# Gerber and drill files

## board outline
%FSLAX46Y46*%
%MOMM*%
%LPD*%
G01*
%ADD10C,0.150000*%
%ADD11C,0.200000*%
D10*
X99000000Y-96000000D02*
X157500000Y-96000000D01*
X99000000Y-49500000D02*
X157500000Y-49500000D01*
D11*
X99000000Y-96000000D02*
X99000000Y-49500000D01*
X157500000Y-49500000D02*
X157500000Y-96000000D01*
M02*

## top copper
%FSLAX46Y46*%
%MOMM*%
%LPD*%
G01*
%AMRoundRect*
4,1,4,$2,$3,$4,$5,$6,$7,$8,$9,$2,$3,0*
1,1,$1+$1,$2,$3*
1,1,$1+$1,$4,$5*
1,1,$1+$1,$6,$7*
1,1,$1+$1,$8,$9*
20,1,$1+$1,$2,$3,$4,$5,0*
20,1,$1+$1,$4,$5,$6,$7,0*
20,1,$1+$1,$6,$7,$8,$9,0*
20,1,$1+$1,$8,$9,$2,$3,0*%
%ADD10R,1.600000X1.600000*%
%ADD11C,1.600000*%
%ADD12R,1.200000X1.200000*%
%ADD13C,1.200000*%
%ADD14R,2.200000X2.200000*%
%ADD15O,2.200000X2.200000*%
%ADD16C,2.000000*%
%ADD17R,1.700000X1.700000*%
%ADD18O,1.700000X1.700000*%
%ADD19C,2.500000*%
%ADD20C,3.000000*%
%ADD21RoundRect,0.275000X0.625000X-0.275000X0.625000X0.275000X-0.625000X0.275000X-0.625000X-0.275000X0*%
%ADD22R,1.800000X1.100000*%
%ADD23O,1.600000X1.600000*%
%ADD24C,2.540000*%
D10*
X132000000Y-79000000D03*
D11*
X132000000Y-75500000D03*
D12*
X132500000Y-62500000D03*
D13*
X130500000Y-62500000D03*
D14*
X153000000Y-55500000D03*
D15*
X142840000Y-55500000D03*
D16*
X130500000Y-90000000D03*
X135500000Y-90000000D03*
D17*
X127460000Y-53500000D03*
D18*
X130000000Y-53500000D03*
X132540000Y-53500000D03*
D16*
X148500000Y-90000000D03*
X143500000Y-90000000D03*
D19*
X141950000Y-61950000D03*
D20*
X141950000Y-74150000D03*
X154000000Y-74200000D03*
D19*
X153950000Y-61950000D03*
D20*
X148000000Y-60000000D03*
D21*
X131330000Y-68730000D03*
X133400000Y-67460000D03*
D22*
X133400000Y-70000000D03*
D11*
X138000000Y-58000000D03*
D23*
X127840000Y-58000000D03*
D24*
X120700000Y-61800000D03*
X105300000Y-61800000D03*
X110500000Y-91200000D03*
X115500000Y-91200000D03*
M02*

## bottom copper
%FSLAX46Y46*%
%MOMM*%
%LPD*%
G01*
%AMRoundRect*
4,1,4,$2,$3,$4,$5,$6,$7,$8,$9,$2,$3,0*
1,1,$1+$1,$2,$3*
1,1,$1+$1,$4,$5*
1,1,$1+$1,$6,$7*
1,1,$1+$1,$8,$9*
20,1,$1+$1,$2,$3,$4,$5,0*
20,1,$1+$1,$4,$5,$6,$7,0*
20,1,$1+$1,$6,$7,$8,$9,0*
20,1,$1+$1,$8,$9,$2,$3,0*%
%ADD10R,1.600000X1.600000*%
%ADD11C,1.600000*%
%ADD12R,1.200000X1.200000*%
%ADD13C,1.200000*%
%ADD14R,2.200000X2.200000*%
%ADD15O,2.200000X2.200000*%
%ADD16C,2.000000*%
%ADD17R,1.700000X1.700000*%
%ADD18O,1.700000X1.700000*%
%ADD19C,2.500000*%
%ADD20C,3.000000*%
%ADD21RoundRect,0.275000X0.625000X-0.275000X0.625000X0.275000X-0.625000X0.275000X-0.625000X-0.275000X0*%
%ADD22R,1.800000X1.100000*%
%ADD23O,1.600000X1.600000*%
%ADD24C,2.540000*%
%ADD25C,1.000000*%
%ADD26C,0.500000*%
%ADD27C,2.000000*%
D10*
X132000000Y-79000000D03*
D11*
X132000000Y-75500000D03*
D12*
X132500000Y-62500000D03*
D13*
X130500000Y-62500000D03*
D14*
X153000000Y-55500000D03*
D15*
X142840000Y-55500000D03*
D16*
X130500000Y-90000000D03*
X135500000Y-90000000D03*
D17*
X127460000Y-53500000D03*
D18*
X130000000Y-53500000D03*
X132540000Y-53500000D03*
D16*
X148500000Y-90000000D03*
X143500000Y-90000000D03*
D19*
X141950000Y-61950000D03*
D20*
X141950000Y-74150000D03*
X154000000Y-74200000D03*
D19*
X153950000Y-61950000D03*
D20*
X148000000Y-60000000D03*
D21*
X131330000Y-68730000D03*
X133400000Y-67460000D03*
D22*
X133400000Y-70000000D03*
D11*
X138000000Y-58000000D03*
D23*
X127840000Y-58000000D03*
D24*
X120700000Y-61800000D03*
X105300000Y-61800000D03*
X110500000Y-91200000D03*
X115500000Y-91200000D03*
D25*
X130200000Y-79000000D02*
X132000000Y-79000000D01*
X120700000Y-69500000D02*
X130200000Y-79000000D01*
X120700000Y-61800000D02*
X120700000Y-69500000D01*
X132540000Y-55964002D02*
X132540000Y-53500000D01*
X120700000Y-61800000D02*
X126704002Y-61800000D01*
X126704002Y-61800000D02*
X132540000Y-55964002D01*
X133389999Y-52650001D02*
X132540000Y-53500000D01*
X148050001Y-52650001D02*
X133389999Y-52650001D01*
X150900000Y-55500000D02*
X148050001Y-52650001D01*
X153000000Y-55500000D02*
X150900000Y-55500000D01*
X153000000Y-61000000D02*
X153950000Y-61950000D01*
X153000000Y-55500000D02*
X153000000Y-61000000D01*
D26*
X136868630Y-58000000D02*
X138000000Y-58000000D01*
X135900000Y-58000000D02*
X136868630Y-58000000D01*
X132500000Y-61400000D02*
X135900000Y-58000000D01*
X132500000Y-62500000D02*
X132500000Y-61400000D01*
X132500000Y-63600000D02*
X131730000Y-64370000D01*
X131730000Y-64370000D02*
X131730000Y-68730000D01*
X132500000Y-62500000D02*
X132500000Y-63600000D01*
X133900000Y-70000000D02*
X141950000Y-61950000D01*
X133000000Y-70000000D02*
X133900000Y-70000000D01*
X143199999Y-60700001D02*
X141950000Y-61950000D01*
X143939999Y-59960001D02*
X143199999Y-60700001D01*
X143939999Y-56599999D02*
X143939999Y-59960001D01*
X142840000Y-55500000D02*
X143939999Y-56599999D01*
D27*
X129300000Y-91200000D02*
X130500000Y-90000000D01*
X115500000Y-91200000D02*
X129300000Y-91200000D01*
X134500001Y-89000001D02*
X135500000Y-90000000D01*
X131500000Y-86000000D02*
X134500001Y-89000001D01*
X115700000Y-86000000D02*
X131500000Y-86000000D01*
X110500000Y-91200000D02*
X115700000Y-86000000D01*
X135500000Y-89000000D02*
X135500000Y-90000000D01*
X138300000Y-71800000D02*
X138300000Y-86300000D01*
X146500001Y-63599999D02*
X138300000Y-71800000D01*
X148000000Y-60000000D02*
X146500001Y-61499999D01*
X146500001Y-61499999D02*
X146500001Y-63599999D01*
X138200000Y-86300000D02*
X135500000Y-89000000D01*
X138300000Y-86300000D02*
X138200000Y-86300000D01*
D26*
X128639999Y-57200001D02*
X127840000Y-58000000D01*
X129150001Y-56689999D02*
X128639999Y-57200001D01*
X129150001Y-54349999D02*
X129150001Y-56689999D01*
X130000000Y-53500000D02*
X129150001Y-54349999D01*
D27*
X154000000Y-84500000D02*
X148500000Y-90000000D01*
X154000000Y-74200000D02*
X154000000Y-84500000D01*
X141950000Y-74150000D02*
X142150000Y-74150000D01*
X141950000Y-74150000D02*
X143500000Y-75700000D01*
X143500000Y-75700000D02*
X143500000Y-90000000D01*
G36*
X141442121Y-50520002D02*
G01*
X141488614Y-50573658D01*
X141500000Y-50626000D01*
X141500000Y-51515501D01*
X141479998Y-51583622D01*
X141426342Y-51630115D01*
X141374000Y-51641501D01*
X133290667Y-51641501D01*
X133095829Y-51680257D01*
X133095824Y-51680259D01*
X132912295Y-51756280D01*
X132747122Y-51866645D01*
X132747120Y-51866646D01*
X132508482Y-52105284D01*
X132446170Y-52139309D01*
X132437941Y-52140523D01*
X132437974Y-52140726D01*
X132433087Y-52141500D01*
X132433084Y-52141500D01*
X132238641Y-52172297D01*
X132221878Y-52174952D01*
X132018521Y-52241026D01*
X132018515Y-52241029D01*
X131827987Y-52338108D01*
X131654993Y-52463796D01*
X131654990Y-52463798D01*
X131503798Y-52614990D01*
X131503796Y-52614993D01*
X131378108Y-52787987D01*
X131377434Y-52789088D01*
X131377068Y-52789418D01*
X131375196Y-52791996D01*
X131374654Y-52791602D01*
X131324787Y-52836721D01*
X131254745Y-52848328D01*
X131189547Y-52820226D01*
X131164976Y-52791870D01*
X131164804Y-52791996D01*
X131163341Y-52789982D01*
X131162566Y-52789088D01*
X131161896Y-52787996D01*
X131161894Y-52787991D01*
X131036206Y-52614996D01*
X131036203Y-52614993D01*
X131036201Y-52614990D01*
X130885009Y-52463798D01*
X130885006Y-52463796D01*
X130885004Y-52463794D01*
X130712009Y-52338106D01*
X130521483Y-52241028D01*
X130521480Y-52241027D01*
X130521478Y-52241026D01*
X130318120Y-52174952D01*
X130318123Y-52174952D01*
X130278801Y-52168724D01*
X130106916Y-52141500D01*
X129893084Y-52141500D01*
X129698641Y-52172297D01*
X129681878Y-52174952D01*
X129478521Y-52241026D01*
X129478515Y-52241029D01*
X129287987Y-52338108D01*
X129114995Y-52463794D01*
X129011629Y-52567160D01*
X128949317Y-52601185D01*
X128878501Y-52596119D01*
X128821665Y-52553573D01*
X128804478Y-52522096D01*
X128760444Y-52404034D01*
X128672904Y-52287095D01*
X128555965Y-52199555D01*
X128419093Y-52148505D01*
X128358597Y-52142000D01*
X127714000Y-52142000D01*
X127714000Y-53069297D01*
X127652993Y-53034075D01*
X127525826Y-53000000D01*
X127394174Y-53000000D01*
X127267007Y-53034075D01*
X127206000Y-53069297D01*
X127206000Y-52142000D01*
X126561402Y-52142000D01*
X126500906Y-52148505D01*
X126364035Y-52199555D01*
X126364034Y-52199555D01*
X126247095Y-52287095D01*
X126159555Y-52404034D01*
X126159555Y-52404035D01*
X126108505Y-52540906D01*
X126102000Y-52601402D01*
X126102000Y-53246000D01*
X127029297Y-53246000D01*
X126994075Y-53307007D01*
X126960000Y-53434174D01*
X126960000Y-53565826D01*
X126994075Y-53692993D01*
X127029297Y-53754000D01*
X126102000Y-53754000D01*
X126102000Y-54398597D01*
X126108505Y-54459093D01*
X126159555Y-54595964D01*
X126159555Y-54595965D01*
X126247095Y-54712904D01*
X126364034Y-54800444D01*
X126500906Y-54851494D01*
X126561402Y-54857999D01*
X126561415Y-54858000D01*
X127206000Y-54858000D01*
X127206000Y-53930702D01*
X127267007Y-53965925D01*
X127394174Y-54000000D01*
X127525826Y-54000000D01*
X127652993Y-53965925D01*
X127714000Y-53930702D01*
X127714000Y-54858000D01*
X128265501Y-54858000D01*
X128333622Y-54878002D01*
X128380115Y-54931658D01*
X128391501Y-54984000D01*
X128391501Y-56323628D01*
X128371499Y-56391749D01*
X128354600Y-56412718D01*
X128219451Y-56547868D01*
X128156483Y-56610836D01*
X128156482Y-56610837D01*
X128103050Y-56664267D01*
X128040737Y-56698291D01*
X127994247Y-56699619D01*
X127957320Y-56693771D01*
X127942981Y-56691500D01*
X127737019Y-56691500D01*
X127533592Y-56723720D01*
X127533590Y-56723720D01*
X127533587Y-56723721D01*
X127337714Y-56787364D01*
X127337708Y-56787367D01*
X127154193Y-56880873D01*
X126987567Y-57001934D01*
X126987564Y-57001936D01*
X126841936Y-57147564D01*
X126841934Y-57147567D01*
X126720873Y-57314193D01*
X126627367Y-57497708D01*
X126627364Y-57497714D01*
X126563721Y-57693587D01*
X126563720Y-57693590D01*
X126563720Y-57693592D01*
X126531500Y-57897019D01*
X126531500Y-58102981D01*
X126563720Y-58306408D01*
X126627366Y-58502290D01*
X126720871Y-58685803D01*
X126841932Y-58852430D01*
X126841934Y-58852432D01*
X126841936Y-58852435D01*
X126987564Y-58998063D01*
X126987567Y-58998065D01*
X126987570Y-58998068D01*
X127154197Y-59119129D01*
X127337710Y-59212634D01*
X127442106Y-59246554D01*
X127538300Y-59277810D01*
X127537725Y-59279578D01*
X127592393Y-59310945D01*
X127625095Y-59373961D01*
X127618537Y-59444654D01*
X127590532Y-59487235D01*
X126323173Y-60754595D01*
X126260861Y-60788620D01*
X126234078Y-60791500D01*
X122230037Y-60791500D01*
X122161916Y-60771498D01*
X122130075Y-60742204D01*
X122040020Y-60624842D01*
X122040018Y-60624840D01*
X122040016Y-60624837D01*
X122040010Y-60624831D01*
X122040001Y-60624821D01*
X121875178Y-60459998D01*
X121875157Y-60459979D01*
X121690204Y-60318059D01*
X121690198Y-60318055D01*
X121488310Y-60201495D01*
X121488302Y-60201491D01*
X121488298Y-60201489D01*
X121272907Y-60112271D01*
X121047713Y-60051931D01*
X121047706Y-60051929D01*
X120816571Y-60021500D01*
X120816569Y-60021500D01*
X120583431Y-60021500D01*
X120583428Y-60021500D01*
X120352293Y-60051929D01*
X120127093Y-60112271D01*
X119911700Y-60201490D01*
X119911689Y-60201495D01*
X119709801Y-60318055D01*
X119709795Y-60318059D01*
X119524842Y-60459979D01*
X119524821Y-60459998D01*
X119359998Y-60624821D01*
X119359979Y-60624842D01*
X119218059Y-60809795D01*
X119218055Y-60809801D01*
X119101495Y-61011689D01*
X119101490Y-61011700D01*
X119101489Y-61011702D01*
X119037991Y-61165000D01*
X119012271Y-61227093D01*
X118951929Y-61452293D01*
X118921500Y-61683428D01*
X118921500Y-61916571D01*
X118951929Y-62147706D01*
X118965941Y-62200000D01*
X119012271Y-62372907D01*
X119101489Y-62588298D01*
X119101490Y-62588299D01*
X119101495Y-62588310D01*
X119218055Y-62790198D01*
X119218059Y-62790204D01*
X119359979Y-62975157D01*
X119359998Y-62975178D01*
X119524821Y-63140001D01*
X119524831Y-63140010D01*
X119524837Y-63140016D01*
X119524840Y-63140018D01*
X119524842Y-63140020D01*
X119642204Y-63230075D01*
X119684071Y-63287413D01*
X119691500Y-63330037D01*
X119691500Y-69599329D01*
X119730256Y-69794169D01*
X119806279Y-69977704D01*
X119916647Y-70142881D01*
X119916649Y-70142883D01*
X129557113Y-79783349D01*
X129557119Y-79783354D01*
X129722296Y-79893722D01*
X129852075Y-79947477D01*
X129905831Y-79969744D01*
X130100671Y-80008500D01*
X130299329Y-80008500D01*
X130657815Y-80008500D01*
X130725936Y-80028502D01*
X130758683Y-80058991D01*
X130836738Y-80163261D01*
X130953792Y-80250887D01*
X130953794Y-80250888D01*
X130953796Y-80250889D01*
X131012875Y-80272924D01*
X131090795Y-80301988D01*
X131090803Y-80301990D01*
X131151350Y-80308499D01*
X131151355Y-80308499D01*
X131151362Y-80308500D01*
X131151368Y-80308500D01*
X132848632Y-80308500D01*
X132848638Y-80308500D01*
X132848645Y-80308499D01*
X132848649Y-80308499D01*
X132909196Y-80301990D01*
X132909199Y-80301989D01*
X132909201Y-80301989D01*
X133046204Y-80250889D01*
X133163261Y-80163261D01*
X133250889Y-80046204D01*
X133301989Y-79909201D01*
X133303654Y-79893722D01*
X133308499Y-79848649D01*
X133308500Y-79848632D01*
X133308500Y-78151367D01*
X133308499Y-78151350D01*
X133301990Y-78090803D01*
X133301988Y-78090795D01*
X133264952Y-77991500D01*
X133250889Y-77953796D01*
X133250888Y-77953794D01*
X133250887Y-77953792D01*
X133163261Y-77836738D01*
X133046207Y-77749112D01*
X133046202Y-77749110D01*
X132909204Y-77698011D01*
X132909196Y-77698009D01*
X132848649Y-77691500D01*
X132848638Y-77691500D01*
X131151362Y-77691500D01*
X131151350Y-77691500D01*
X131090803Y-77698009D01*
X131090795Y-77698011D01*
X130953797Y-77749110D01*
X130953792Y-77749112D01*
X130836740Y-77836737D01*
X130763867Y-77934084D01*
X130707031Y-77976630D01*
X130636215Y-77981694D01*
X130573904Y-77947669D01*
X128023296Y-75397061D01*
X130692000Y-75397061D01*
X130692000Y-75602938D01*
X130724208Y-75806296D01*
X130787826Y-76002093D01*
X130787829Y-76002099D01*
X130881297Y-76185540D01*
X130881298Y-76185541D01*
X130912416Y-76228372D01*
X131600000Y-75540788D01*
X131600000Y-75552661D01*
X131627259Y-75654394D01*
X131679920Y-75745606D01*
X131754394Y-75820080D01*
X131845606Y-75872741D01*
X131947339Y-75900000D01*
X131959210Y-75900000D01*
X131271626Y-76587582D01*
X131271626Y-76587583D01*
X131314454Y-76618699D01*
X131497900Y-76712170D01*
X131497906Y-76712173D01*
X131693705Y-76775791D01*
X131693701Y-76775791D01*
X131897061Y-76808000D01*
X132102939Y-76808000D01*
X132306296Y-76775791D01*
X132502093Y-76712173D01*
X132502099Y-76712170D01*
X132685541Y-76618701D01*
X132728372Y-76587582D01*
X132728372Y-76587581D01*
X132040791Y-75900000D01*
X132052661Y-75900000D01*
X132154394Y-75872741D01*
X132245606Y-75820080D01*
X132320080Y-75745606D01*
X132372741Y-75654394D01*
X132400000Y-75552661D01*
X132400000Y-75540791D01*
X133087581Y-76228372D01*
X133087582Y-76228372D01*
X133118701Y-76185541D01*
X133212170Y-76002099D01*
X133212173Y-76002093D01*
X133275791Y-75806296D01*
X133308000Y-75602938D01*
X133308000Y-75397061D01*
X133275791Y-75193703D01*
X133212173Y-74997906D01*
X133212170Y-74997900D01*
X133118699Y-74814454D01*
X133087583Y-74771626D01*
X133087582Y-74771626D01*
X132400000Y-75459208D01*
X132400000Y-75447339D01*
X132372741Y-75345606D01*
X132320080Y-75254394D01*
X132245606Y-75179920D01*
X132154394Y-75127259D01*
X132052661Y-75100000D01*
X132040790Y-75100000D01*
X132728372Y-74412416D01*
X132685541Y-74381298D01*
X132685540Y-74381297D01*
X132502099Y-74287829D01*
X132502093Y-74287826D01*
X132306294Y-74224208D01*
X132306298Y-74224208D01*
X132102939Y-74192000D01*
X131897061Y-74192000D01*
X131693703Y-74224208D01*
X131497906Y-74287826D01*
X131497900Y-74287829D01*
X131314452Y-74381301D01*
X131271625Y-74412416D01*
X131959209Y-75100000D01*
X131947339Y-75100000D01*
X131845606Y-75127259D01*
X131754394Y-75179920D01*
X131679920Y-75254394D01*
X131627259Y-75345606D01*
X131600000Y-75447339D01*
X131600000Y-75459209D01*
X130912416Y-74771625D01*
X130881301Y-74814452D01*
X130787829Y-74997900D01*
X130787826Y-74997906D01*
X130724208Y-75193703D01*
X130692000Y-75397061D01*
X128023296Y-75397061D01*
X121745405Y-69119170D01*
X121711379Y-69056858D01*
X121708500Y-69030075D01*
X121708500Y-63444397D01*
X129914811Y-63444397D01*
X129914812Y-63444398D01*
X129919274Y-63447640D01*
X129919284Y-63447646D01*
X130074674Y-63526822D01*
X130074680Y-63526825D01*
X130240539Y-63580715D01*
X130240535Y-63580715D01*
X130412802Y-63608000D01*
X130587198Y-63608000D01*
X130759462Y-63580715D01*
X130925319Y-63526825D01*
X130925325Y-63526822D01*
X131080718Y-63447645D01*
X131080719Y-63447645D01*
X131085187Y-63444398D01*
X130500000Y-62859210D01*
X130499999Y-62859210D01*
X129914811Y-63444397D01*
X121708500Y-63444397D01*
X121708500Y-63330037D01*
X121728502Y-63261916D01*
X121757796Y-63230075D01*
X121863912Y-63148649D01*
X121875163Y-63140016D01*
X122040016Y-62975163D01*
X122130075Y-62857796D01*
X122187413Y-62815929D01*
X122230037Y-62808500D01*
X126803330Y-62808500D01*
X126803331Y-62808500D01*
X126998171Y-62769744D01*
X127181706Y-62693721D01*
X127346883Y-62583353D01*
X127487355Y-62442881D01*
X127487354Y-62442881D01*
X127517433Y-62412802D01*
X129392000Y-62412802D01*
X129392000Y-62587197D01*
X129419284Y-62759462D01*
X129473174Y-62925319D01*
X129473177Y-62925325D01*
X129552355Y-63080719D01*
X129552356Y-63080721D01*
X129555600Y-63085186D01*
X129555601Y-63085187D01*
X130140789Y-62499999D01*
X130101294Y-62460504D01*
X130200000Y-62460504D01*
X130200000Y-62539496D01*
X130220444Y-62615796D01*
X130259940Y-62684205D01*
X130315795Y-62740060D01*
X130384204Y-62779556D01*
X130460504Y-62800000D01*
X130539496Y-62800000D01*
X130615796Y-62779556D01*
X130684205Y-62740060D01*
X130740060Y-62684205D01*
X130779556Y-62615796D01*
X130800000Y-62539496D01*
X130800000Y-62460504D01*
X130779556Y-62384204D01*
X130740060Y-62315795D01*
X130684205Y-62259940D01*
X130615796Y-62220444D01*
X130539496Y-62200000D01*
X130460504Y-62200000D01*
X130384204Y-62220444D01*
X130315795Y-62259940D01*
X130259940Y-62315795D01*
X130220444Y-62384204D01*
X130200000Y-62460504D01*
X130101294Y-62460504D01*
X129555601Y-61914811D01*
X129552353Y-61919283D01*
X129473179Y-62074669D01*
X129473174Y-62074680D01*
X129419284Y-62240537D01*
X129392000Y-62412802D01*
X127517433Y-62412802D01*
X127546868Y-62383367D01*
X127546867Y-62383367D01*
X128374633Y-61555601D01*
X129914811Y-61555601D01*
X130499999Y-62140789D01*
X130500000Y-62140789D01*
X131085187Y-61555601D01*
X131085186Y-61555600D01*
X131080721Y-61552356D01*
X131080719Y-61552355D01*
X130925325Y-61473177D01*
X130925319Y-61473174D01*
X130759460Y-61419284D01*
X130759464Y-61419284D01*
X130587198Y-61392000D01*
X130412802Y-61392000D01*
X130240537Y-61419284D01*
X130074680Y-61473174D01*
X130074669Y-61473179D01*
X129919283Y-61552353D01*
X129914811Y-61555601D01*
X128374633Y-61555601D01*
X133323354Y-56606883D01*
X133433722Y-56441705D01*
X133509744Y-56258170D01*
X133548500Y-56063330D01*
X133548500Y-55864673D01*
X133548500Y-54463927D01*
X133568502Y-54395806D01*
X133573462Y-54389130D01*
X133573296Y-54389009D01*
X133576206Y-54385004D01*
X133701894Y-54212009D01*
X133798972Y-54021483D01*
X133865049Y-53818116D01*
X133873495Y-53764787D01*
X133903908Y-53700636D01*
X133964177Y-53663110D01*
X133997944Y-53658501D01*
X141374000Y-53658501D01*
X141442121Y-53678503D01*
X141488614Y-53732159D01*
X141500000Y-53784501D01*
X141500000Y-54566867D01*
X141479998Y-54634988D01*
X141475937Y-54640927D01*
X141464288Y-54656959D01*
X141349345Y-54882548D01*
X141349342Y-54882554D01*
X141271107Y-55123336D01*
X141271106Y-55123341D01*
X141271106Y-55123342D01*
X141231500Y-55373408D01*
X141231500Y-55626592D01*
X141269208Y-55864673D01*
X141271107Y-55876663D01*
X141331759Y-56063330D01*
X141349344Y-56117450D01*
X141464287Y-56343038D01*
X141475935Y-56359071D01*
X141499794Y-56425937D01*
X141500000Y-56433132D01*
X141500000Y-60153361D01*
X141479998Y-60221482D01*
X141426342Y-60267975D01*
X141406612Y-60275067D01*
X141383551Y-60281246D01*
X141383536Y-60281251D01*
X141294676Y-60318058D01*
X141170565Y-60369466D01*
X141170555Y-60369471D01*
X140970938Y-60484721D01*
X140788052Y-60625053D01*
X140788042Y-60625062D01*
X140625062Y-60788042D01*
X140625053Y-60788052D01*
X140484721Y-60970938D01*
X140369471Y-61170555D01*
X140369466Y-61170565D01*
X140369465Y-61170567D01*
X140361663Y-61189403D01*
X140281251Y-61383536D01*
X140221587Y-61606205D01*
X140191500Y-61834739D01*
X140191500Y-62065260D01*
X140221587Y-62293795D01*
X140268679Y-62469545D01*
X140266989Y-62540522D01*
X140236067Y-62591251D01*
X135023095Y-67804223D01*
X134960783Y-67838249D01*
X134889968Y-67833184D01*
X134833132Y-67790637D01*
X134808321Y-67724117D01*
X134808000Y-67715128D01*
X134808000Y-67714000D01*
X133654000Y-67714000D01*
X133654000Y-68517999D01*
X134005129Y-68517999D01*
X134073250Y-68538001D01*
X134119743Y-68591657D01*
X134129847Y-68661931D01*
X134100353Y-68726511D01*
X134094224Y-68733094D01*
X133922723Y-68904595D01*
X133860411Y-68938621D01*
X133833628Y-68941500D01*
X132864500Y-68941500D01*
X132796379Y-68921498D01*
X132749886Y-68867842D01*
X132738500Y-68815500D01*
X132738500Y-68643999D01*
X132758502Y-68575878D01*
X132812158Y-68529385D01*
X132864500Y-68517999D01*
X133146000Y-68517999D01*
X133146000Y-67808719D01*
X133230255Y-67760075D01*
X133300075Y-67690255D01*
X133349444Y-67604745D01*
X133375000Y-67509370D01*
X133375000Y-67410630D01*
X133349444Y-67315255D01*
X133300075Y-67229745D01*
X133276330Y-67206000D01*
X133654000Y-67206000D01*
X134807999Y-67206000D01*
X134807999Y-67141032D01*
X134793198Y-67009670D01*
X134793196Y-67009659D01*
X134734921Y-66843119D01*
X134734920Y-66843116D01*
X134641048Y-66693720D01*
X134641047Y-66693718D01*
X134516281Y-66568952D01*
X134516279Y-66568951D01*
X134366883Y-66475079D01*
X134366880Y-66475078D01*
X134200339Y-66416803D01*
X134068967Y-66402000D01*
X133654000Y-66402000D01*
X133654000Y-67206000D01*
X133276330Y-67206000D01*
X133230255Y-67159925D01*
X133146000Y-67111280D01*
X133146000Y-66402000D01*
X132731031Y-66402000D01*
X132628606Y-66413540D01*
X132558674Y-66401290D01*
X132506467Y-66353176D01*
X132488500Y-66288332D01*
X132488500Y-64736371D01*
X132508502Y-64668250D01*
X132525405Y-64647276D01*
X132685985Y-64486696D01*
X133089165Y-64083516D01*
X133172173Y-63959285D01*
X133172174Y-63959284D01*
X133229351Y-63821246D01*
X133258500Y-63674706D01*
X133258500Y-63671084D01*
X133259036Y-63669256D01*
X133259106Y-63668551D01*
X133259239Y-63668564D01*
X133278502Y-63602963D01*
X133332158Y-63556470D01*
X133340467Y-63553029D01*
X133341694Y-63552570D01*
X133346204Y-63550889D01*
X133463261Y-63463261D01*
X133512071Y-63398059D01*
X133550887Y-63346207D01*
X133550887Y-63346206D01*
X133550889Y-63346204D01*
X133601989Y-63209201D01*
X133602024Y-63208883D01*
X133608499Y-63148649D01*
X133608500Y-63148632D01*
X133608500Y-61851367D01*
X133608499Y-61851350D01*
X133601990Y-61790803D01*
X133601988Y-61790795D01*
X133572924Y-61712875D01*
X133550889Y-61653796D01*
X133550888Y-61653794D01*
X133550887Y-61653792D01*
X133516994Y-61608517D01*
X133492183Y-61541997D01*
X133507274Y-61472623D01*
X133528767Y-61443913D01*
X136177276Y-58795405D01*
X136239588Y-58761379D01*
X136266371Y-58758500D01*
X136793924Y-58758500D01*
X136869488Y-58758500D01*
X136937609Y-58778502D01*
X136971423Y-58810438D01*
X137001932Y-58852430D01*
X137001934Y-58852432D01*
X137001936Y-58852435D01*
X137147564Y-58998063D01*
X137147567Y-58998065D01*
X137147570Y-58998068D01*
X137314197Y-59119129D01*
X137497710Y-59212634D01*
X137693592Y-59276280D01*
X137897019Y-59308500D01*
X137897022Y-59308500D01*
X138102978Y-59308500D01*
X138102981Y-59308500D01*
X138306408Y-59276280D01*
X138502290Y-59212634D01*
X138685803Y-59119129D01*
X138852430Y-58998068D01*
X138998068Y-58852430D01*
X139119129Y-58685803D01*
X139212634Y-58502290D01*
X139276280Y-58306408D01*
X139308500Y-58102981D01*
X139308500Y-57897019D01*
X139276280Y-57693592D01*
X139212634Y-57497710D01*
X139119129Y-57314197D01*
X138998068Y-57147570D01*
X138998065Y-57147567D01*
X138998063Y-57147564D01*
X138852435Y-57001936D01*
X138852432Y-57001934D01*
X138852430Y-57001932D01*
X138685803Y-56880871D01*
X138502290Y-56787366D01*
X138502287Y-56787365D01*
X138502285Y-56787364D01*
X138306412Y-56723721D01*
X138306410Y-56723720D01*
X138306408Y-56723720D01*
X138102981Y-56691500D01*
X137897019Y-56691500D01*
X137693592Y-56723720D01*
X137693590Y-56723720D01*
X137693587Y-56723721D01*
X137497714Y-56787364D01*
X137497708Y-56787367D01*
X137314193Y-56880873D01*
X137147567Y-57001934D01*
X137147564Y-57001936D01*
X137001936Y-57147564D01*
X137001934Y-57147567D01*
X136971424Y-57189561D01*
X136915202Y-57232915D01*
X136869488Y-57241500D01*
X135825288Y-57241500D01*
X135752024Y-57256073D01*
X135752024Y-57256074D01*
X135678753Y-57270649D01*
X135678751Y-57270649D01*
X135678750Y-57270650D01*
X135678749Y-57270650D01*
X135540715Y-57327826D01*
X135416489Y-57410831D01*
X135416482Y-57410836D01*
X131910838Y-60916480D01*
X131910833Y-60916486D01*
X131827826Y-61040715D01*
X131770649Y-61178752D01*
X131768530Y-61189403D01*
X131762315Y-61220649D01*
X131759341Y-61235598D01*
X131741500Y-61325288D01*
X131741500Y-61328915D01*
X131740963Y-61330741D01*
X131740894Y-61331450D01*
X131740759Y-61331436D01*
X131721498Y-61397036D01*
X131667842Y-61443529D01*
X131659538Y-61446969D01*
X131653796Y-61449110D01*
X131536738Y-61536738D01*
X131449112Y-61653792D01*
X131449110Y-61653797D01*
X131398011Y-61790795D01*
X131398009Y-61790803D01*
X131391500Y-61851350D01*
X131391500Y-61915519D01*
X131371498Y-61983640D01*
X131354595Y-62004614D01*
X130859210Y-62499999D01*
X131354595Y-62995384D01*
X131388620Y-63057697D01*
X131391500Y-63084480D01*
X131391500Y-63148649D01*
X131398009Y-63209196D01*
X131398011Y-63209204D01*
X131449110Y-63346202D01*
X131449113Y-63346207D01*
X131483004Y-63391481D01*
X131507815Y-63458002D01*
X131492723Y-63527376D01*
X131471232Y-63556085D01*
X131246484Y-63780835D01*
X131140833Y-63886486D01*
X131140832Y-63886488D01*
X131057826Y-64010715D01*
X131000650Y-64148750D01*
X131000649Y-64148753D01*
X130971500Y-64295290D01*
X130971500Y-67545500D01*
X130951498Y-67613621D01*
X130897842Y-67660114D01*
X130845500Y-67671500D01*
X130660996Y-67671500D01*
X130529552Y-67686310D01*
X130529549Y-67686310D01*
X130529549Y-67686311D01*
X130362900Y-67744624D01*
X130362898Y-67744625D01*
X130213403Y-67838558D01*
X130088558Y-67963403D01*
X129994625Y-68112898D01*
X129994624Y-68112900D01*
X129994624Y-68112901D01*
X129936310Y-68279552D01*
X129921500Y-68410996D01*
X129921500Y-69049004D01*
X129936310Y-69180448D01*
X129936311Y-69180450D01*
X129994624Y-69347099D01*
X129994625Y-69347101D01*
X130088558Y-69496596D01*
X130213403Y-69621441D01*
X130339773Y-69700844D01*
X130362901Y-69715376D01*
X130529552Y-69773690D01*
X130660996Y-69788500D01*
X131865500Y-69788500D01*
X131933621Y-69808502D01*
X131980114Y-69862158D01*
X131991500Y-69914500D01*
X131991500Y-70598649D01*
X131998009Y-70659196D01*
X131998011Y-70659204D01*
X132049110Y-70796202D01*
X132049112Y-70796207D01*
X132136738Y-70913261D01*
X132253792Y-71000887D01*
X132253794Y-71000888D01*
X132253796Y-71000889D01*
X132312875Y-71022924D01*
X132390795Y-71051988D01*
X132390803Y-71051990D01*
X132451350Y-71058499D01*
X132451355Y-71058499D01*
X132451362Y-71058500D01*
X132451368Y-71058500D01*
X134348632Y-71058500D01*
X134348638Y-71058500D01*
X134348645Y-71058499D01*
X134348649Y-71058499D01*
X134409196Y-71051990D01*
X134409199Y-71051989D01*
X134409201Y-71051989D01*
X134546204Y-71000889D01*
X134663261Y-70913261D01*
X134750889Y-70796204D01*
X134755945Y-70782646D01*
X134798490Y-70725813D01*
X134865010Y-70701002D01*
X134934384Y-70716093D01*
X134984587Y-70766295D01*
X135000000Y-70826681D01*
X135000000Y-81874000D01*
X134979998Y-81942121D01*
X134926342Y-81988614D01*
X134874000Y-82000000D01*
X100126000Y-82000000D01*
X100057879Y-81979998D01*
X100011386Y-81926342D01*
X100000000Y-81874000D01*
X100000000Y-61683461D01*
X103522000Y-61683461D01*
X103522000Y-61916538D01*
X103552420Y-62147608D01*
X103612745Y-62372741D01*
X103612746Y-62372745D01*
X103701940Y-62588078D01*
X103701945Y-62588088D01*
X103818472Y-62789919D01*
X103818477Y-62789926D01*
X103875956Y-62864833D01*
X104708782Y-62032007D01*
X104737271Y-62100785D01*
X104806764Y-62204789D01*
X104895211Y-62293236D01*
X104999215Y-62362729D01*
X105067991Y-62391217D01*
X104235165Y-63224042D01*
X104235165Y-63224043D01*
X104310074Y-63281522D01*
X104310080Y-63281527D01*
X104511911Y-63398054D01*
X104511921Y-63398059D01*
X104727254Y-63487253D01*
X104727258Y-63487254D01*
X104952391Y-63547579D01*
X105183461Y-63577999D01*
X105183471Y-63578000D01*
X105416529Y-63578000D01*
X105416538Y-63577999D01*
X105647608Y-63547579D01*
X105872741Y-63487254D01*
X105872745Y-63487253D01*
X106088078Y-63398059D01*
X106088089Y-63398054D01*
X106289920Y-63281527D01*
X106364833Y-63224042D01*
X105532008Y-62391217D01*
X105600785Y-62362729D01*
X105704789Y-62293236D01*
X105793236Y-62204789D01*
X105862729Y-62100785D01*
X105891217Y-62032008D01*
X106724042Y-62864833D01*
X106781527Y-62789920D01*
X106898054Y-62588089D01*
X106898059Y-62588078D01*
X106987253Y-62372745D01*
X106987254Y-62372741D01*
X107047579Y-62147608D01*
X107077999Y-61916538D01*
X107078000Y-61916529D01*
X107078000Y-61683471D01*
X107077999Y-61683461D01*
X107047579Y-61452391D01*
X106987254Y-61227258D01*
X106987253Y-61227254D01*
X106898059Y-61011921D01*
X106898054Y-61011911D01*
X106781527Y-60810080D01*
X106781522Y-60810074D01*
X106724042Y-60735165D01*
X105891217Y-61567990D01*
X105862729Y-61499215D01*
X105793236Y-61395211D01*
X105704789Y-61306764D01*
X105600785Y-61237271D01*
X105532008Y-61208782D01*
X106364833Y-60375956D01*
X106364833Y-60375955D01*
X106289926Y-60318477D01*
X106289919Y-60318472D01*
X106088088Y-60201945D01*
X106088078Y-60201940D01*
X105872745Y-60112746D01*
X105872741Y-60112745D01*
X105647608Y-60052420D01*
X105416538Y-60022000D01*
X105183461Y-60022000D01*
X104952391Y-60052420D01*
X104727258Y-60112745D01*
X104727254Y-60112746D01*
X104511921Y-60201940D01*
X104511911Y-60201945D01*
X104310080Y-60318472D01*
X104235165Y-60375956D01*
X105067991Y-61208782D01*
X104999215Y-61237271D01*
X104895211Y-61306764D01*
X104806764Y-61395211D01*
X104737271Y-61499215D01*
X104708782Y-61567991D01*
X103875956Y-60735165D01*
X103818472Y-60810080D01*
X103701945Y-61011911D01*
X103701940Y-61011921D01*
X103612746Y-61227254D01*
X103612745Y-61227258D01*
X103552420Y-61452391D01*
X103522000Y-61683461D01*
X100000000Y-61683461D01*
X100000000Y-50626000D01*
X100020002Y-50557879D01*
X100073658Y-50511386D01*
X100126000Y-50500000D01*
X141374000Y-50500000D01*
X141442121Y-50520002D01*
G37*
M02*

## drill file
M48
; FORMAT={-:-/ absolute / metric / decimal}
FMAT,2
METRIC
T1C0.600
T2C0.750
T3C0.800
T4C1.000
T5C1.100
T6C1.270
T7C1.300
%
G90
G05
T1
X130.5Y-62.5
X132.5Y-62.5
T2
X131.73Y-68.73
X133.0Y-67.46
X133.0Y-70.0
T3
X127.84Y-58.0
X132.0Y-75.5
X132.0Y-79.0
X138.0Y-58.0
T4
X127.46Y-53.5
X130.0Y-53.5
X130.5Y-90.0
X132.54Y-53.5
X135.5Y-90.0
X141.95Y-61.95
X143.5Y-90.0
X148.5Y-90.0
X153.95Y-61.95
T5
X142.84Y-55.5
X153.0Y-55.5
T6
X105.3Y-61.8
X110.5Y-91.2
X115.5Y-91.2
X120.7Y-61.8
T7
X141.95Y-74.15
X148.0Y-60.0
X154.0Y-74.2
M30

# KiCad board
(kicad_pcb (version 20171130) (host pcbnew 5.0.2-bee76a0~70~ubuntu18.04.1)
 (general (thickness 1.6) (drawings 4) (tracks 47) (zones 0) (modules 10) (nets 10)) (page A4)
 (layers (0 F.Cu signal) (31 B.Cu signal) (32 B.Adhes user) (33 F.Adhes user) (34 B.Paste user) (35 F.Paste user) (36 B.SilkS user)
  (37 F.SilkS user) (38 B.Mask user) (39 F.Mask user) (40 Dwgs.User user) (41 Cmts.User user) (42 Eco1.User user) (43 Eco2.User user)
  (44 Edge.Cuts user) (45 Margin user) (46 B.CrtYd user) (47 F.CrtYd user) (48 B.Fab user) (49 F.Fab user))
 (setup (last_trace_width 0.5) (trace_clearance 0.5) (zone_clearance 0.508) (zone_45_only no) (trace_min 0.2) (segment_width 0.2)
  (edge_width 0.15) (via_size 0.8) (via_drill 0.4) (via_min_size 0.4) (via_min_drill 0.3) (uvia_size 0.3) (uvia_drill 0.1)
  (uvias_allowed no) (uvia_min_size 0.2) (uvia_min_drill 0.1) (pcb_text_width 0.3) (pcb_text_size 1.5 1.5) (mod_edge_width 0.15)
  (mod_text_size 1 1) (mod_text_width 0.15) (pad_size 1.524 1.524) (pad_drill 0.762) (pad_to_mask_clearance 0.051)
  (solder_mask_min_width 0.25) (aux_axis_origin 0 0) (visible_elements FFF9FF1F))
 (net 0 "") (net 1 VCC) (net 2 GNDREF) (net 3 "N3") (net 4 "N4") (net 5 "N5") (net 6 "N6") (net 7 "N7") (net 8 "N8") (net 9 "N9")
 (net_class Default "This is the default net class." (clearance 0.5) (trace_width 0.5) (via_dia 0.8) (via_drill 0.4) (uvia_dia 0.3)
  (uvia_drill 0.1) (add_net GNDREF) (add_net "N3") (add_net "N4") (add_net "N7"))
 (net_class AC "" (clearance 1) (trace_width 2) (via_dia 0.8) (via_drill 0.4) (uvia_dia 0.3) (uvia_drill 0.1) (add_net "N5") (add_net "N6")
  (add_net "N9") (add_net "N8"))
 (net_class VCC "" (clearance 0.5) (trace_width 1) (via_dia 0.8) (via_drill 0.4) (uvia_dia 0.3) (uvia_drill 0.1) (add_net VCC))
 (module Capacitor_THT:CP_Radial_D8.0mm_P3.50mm (layer F.Cu) (at 132 79 90)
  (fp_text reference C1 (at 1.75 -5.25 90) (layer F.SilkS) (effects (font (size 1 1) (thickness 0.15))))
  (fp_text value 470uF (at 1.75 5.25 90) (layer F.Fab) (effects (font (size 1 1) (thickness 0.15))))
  (pad 1 thru_hole rect (at 0 0 90) (size 1.6 1.6) (drill 0.8) (layers *.Cu *.Mask) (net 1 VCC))
  (pad 2 thru_hole circle (at 3.5 0 90) (size 1.6 1.6) (drill 0.8) (layers *.Cu *.Mask) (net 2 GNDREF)))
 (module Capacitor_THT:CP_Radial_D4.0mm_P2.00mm (layer F.Cu) (at 132.5 62.5 180)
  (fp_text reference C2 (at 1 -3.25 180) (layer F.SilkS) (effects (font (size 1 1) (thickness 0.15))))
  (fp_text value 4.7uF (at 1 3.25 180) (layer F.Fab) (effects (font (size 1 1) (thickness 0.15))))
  (pad 1 thru_hole rect (at 0 0 180) (size 1.2 1.2) (drill 0.6) (layers *.Cu *.Mask) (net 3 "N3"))
  (pad 2 thru_hole circle (at 2 0 180) (size 1.2 1.2) (drill 0.6) (layers *.Cu *.Mask) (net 2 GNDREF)))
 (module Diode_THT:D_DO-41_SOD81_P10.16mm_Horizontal (layer F.Cu) (at 153 55.5 180)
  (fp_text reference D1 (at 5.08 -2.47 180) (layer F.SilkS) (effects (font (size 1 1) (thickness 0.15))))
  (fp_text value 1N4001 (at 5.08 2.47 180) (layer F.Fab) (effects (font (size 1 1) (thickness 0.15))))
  (pad 1 thru_hole rect (at 0 0 180) (size 2.2 2.2) (drill 1.1) (layers *.Cu *.Mask) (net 1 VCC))
  (pad 2 thru_hole oval (at 10.16 0 180) (size 2.2 2.2) (drill 1.1) (layers *.Cu *.Mask) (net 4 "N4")))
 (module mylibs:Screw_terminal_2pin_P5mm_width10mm (layer F.Cu) (at 128 95)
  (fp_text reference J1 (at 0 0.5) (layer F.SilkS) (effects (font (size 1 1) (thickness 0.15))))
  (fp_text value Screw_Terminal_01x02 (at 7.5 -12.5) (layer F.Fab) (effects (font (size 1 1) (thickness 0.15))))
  (pad 1 thru_hole circle (at 2.5 -5) (size 2 2) (drill 1) (layers *.Cu *.Mask) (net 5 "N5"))
  (pad 2 thru_hole circle (at 7.5 -5) (size 2 2) (drill 1) (layers *.Cu *.Mask) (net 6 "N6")))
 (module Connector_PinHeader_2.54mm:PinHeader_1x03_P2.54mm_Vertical (layer F.Cu) (at 127.46 53.5 90)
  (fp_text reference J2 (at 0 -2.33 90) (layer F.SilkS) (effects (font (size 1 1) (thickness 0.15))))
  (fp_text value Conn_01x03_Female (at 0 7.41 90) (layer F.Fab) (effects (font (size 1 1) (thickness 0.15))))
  (pad 1 thru_hole rect (at 0 0 90) (size 1.7 1.7) (drill 1) (layers *.Cu *.Mask) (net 2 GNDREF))
  (pad 2 thru_hole oval (at 0 2.54 90) (size 1.7 1.7) (drill 1) (layers *.Cu *.Mask) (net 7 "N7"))
  (pad 3 thru_hole oval (at 0 5.08 90) (size 1.7 1.7) (drill 1) (layers *.Cu *.Mask) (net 1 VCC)))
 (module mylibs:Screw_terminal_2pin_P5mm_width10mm (layer F.Cu) (at 141 95)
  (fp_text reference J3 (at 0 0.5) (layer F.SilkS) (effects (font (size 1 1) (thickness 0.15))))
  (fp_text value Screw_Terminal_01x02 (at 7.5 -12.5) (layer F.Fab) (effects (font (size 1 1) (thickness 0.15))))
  (pad 2 thru_hole circle (at 7.5 -5) (size 2 2) (drill 1) (layers *.Cu *.Mask) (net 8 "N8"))
  (pad 1 thru_hole circle (at 2.5 -5) (size 2 2) (drill 1) (layers *.Cu *.Mask) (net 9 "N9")))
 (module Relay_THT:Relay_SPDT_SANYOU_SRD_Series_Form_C (layer F.Cu) (at 148 60 270)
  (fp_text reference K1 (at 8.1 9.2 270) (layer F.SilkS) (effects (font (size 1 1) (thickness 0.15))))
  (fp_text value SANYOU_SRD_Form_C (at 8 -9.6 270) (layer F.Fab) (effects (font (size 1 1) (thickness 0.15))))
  (pad 2 thru_hole circle (at 1.95 6.05) (size 2.5 2.5) (drill 1) (layers *.Cu *.Mask) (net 4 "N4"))
  (pad 3 thru_hole circle (at 14.15 6.05) (size 3 3) (drill 1.3) (layers *.Cu *.Mask) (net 9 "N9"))
  (pad 4 thru_hole circle (at 14.2 -6) (size 3 3) (drill 1.3) (layers *.Cu *.Mask) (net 8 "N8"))
  (pad 5 thru_hole circle (at 1.95 -5.95) (size 2.5 2.5) (drill 1) (layers *.Cu *.Mask) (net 1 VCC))
  (pad 1 thru_hole circle (at 0 0) (size 3 3) (drill 1.3) (layers *.Cu *.Mask) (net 6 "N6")))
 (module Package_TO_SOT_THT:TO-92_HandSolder (layer F.Cu) (at 133 70 90)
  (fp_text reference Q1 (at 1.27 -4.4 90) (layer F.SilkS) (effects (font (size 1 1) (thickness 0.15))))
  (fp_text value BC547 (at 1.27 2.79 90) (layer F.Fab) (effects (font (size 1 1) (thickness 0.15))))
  (pad 2 thru_hole roundrect (at 1.27 -1.27 90) (size 1.1 1.8) (drill 0.75 (offset 0 -0.4)) (layers *.Cu *.Mask) (roundrect_rratio 0.25)
   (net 3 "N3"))
  (pad 3 thru_hole roundrect (at 2.54 0 90) (size 1.1 1.8) (drill 0.75 (offset 0 0.4)) (layers *.Cu *.Mask) (roundrect_rratio 0.25)
   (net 2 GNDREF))
  (pad 1 thru_hole rect (at 0 0 90) (size 1.1 1.8) (drill 0.75 (offset 0 0.4)) (layers *.Cu *.Mask) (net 4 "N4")))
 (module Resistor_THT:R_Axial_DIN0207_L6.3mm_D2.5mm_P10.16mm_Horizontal (layer F.Cu) (at 138 58 180)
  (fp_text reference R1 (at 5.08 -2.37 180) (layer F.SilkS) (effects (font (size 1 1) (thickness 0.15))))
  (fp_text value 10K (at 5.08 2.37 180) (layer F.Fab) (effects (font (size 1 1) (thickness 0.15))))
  (pad 1 thru_hole circle (at 0 0 180) (size 1.6 1.6) (drill 0.8) (layers *.Cu *.Mask) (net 3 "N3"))
  (pad 2 thru_hole oval (at 10.16 0 180) (size 1.6 1.6) (drill 0.8) (layers *.Cu *.Mask) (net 7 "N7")))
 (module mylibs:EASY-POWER (layer F.Cu) (at 125 95 90)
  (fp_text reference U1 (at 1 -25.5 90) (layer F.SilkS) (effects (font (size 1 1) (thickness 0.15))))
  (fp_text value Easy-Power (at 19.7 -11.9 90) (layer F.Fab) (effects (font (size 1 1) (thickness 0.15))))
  (pad 4 thru_hole circle (at 33.2 -4.3 90) (size 2.54 2.54) (drill 1.27) (layers *.Cu *.Mask) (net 1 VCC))
  (pad 3 thru_hole circle (at 33.2 -19.7 90) (size 2.54 2.54) (drill 1.27) (layers *.Cu *.Mask) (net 2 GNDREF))
  (pad 1 thru_hole circle (at 3.8 -14.5 90) (size 2.54 2.54) (drill 1.27) (layers *.Cu *.Mask) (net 6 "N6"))
  (pad 2 thru_hole circle (at 3.8 -9.5 90) (size 2.54 2.54) (drill 1.27) (layers *.Cu *.Mask) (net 5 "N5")))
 (gr_line (start 99 96) (end 157.5 96) (layer Edge.Cuts) (width 0.15))
 (gr_line (start 99 49.5) (end 157.5 49.5) (layer Edge.Cuts) (width 0.15))
 (gr_line (start 99 96) (end 99 49.5) (layer Edge.Cuts) (width 0.2))
 (gr_line (start 157.5 49.5) (end 157.5 96) (layer Edge.Cuts) (width 0.2))
 (segment (start 130.2 79) (end 132 79) (width 1) (layer B.Cu) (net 1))
 (segment (start 120.7 69.5) (end 130.2 79) (width 1) (layer B.Cu) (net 1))
 (segment (start 120.7 61.8) (end 120.7 69.5) (width 1) (layer B.Cu) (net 1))
 (segment (start 132.54 55.964002) (end 132.54 53.5) (width 1) (layer B.Cu) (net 1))
 (segment (start 120.7 61.8) (end 126.704002 61.8) (width 1) (layer B.Cu) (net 1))
 (segment (start 126.704002 61.8) (end 132.54 55.964002) (width 1) (layer B.Cu) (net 1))
 (segment (start 133.389999 52.650001) (end 132.54 53.5) (width 1) (layer B.Cu) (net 1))
 (segment (start 148.050001 52.650001) (end 133.389999 52.650001) (width 1) (layer B.Cu) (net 1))
 (segment (start 150.9 55.5) (end 148.050001 52.650001) (width 1) (layer B.Cu) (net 1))
 (segment (start 153 55.5) (end 150.9 55.5) (width 1) (layer B.Cu) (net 1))
 (segment (start 153 61) (end 153.95 61.95) (width 1) (layer B.Cu) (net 1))
 (segment (start 153 55.5) (end 153 61) (width 1) (layer B.Cu) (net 1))
 (segment (start 136.86863 58) (end 138 58) (width 0.5) (layer B.Cu) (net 3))
 (segment (start 135.9 58) (end 136.86863 58) (width 0.5) (layer B.Cu) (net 3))
 (segment (start 132.5 61.4) (end 135.9 58) (width 0.5) (layer B.Cu) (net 3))
 (segment (start 132.5 62.5) (end 132.5 61.4) (width 0.5) (layer B.Cu) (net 3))
 (segment (start 132.5 63.6) (end 131.73 64.37) (width 0.5) (layer B.Cu) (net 3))
 (segment (start 131.73 64.37) (end 131.73 68.73) (width 0.5) (layer B.Cu) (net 3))
 (segment (start 132.5 62.5) (end 132.5 63.6) (width 0.5) (layer B.Cu) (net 3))
 (segment (start 133.9 70) (end 141.95 61.95) (width 0.5) (layer B.Cu) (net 4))
 (segment (start 133 70) (end 133.9 70) (width 0.5) (layer B.Cu) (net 4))
 (segment (start 143.199999 60.700001) (end 141.95 61.95) (width 0.5) (layer B.Cu) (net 4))
 (segment (start 143.939999 59.960001) (end 143.199999 60.700001) (width 0.5) (layer B.Cu) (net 4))
 (segment (start 143.939999 56.599999) (end 143.939999 59.960001) (width 0.5) (layer B.Cu) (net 4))
 (segment (start 142.84 55.5) (end 143.939999 56.599999) (width 0.5) (layer B.Cu) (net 4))
 (segment (start 129.3 91.2) (end 130.5 90) (width 2) (layer B.Cu) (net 5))
 (segment (start 115.5 91.2) (end 129.3 91.2) (width 2) (layer B.Cu) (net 5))
 (segment (start 134.500001 89.000001) (end 135.5 90) (width 2) (layer B.Cu) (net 6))
 (segment (start 131.5 86) (end 134.500001 89.000001) (width 2) (layer B.Cu) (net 6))
 (segment (start 115.7 86) (end 131.5 86) (width 2) (layer B.Cu) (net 6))
 (segment (start 110.5 91.2) (end 115.7 86) (width 2) (layer B.Cu) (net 6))
 (segment (start 135.5 89) (end 135.5 90) (width 2) (layer B.Cu) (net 6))
 (segment (start 138.3 71.8) (end 138.3 86.3) (width 2) (layer B.Cu) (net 6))
 (segment (start 146.500001 63.599999) (end 138.3 71.8) (width 2) (layer B.Cu) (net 6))
 (segment (start 148 60) (end 146.500001 61.499999) (width 2) (layer B.Cu) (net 6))
 (segment (start 146.500001 61.499999) (end 146.500001 63.599999) (width 2) (layer B.Cu) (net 6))
 (segment (start 138.2 86.3) (end 135.5 89) (width 2) (layer B.Cu) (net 6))
 (segment (start 138.3 86.3) (end 138.2 86.3) (width 2) (layer B.Cu) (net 6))
 (segment (start 128.639999 57.200001) (end 127.84 58) (width 0.5) (layer B.Cu) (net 7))
 (segment (start 129.150001 56.689999) (end 128.639999 57.200001) (width 0.5) (layer B.Cu) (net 7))
 (segment (start 129.150001 54.349999) (end 129.150001 56.689999) (width 0.5) (layer B.Cu) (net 7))
 (segment (start 130 53.5) (end 129.150001 54.349999) (width 0.5) (layer B.Cu) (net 7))
 (segment (start 154 84.5) (end 148.5 90) (width 2) (layer B.Cu) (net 8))
 (segment (start 154 74.2) (end 154 84.5) (width 2) (layer B.Cu) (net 8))
 (segment (start 141.95 74.15) (end 142.15 74.15) (width 2) (layer B.Cu) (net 9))
 (segment (start 141.95 74.15) (end 143.5 75.7) (width 2) (layer B.Cu) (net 9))
 (segment (start 143.5 75.7) (end 143.5 90) (width 2) (layer B.Cu) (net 9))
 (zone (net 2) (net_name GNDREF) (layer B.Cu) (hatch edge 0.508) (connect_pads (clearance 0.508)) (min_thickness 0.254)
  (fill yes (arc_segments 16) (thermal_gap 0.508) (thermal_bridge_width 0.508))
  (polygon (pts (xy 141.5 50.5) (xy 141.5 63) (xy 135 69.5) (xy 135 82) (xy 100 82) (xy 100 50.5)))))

